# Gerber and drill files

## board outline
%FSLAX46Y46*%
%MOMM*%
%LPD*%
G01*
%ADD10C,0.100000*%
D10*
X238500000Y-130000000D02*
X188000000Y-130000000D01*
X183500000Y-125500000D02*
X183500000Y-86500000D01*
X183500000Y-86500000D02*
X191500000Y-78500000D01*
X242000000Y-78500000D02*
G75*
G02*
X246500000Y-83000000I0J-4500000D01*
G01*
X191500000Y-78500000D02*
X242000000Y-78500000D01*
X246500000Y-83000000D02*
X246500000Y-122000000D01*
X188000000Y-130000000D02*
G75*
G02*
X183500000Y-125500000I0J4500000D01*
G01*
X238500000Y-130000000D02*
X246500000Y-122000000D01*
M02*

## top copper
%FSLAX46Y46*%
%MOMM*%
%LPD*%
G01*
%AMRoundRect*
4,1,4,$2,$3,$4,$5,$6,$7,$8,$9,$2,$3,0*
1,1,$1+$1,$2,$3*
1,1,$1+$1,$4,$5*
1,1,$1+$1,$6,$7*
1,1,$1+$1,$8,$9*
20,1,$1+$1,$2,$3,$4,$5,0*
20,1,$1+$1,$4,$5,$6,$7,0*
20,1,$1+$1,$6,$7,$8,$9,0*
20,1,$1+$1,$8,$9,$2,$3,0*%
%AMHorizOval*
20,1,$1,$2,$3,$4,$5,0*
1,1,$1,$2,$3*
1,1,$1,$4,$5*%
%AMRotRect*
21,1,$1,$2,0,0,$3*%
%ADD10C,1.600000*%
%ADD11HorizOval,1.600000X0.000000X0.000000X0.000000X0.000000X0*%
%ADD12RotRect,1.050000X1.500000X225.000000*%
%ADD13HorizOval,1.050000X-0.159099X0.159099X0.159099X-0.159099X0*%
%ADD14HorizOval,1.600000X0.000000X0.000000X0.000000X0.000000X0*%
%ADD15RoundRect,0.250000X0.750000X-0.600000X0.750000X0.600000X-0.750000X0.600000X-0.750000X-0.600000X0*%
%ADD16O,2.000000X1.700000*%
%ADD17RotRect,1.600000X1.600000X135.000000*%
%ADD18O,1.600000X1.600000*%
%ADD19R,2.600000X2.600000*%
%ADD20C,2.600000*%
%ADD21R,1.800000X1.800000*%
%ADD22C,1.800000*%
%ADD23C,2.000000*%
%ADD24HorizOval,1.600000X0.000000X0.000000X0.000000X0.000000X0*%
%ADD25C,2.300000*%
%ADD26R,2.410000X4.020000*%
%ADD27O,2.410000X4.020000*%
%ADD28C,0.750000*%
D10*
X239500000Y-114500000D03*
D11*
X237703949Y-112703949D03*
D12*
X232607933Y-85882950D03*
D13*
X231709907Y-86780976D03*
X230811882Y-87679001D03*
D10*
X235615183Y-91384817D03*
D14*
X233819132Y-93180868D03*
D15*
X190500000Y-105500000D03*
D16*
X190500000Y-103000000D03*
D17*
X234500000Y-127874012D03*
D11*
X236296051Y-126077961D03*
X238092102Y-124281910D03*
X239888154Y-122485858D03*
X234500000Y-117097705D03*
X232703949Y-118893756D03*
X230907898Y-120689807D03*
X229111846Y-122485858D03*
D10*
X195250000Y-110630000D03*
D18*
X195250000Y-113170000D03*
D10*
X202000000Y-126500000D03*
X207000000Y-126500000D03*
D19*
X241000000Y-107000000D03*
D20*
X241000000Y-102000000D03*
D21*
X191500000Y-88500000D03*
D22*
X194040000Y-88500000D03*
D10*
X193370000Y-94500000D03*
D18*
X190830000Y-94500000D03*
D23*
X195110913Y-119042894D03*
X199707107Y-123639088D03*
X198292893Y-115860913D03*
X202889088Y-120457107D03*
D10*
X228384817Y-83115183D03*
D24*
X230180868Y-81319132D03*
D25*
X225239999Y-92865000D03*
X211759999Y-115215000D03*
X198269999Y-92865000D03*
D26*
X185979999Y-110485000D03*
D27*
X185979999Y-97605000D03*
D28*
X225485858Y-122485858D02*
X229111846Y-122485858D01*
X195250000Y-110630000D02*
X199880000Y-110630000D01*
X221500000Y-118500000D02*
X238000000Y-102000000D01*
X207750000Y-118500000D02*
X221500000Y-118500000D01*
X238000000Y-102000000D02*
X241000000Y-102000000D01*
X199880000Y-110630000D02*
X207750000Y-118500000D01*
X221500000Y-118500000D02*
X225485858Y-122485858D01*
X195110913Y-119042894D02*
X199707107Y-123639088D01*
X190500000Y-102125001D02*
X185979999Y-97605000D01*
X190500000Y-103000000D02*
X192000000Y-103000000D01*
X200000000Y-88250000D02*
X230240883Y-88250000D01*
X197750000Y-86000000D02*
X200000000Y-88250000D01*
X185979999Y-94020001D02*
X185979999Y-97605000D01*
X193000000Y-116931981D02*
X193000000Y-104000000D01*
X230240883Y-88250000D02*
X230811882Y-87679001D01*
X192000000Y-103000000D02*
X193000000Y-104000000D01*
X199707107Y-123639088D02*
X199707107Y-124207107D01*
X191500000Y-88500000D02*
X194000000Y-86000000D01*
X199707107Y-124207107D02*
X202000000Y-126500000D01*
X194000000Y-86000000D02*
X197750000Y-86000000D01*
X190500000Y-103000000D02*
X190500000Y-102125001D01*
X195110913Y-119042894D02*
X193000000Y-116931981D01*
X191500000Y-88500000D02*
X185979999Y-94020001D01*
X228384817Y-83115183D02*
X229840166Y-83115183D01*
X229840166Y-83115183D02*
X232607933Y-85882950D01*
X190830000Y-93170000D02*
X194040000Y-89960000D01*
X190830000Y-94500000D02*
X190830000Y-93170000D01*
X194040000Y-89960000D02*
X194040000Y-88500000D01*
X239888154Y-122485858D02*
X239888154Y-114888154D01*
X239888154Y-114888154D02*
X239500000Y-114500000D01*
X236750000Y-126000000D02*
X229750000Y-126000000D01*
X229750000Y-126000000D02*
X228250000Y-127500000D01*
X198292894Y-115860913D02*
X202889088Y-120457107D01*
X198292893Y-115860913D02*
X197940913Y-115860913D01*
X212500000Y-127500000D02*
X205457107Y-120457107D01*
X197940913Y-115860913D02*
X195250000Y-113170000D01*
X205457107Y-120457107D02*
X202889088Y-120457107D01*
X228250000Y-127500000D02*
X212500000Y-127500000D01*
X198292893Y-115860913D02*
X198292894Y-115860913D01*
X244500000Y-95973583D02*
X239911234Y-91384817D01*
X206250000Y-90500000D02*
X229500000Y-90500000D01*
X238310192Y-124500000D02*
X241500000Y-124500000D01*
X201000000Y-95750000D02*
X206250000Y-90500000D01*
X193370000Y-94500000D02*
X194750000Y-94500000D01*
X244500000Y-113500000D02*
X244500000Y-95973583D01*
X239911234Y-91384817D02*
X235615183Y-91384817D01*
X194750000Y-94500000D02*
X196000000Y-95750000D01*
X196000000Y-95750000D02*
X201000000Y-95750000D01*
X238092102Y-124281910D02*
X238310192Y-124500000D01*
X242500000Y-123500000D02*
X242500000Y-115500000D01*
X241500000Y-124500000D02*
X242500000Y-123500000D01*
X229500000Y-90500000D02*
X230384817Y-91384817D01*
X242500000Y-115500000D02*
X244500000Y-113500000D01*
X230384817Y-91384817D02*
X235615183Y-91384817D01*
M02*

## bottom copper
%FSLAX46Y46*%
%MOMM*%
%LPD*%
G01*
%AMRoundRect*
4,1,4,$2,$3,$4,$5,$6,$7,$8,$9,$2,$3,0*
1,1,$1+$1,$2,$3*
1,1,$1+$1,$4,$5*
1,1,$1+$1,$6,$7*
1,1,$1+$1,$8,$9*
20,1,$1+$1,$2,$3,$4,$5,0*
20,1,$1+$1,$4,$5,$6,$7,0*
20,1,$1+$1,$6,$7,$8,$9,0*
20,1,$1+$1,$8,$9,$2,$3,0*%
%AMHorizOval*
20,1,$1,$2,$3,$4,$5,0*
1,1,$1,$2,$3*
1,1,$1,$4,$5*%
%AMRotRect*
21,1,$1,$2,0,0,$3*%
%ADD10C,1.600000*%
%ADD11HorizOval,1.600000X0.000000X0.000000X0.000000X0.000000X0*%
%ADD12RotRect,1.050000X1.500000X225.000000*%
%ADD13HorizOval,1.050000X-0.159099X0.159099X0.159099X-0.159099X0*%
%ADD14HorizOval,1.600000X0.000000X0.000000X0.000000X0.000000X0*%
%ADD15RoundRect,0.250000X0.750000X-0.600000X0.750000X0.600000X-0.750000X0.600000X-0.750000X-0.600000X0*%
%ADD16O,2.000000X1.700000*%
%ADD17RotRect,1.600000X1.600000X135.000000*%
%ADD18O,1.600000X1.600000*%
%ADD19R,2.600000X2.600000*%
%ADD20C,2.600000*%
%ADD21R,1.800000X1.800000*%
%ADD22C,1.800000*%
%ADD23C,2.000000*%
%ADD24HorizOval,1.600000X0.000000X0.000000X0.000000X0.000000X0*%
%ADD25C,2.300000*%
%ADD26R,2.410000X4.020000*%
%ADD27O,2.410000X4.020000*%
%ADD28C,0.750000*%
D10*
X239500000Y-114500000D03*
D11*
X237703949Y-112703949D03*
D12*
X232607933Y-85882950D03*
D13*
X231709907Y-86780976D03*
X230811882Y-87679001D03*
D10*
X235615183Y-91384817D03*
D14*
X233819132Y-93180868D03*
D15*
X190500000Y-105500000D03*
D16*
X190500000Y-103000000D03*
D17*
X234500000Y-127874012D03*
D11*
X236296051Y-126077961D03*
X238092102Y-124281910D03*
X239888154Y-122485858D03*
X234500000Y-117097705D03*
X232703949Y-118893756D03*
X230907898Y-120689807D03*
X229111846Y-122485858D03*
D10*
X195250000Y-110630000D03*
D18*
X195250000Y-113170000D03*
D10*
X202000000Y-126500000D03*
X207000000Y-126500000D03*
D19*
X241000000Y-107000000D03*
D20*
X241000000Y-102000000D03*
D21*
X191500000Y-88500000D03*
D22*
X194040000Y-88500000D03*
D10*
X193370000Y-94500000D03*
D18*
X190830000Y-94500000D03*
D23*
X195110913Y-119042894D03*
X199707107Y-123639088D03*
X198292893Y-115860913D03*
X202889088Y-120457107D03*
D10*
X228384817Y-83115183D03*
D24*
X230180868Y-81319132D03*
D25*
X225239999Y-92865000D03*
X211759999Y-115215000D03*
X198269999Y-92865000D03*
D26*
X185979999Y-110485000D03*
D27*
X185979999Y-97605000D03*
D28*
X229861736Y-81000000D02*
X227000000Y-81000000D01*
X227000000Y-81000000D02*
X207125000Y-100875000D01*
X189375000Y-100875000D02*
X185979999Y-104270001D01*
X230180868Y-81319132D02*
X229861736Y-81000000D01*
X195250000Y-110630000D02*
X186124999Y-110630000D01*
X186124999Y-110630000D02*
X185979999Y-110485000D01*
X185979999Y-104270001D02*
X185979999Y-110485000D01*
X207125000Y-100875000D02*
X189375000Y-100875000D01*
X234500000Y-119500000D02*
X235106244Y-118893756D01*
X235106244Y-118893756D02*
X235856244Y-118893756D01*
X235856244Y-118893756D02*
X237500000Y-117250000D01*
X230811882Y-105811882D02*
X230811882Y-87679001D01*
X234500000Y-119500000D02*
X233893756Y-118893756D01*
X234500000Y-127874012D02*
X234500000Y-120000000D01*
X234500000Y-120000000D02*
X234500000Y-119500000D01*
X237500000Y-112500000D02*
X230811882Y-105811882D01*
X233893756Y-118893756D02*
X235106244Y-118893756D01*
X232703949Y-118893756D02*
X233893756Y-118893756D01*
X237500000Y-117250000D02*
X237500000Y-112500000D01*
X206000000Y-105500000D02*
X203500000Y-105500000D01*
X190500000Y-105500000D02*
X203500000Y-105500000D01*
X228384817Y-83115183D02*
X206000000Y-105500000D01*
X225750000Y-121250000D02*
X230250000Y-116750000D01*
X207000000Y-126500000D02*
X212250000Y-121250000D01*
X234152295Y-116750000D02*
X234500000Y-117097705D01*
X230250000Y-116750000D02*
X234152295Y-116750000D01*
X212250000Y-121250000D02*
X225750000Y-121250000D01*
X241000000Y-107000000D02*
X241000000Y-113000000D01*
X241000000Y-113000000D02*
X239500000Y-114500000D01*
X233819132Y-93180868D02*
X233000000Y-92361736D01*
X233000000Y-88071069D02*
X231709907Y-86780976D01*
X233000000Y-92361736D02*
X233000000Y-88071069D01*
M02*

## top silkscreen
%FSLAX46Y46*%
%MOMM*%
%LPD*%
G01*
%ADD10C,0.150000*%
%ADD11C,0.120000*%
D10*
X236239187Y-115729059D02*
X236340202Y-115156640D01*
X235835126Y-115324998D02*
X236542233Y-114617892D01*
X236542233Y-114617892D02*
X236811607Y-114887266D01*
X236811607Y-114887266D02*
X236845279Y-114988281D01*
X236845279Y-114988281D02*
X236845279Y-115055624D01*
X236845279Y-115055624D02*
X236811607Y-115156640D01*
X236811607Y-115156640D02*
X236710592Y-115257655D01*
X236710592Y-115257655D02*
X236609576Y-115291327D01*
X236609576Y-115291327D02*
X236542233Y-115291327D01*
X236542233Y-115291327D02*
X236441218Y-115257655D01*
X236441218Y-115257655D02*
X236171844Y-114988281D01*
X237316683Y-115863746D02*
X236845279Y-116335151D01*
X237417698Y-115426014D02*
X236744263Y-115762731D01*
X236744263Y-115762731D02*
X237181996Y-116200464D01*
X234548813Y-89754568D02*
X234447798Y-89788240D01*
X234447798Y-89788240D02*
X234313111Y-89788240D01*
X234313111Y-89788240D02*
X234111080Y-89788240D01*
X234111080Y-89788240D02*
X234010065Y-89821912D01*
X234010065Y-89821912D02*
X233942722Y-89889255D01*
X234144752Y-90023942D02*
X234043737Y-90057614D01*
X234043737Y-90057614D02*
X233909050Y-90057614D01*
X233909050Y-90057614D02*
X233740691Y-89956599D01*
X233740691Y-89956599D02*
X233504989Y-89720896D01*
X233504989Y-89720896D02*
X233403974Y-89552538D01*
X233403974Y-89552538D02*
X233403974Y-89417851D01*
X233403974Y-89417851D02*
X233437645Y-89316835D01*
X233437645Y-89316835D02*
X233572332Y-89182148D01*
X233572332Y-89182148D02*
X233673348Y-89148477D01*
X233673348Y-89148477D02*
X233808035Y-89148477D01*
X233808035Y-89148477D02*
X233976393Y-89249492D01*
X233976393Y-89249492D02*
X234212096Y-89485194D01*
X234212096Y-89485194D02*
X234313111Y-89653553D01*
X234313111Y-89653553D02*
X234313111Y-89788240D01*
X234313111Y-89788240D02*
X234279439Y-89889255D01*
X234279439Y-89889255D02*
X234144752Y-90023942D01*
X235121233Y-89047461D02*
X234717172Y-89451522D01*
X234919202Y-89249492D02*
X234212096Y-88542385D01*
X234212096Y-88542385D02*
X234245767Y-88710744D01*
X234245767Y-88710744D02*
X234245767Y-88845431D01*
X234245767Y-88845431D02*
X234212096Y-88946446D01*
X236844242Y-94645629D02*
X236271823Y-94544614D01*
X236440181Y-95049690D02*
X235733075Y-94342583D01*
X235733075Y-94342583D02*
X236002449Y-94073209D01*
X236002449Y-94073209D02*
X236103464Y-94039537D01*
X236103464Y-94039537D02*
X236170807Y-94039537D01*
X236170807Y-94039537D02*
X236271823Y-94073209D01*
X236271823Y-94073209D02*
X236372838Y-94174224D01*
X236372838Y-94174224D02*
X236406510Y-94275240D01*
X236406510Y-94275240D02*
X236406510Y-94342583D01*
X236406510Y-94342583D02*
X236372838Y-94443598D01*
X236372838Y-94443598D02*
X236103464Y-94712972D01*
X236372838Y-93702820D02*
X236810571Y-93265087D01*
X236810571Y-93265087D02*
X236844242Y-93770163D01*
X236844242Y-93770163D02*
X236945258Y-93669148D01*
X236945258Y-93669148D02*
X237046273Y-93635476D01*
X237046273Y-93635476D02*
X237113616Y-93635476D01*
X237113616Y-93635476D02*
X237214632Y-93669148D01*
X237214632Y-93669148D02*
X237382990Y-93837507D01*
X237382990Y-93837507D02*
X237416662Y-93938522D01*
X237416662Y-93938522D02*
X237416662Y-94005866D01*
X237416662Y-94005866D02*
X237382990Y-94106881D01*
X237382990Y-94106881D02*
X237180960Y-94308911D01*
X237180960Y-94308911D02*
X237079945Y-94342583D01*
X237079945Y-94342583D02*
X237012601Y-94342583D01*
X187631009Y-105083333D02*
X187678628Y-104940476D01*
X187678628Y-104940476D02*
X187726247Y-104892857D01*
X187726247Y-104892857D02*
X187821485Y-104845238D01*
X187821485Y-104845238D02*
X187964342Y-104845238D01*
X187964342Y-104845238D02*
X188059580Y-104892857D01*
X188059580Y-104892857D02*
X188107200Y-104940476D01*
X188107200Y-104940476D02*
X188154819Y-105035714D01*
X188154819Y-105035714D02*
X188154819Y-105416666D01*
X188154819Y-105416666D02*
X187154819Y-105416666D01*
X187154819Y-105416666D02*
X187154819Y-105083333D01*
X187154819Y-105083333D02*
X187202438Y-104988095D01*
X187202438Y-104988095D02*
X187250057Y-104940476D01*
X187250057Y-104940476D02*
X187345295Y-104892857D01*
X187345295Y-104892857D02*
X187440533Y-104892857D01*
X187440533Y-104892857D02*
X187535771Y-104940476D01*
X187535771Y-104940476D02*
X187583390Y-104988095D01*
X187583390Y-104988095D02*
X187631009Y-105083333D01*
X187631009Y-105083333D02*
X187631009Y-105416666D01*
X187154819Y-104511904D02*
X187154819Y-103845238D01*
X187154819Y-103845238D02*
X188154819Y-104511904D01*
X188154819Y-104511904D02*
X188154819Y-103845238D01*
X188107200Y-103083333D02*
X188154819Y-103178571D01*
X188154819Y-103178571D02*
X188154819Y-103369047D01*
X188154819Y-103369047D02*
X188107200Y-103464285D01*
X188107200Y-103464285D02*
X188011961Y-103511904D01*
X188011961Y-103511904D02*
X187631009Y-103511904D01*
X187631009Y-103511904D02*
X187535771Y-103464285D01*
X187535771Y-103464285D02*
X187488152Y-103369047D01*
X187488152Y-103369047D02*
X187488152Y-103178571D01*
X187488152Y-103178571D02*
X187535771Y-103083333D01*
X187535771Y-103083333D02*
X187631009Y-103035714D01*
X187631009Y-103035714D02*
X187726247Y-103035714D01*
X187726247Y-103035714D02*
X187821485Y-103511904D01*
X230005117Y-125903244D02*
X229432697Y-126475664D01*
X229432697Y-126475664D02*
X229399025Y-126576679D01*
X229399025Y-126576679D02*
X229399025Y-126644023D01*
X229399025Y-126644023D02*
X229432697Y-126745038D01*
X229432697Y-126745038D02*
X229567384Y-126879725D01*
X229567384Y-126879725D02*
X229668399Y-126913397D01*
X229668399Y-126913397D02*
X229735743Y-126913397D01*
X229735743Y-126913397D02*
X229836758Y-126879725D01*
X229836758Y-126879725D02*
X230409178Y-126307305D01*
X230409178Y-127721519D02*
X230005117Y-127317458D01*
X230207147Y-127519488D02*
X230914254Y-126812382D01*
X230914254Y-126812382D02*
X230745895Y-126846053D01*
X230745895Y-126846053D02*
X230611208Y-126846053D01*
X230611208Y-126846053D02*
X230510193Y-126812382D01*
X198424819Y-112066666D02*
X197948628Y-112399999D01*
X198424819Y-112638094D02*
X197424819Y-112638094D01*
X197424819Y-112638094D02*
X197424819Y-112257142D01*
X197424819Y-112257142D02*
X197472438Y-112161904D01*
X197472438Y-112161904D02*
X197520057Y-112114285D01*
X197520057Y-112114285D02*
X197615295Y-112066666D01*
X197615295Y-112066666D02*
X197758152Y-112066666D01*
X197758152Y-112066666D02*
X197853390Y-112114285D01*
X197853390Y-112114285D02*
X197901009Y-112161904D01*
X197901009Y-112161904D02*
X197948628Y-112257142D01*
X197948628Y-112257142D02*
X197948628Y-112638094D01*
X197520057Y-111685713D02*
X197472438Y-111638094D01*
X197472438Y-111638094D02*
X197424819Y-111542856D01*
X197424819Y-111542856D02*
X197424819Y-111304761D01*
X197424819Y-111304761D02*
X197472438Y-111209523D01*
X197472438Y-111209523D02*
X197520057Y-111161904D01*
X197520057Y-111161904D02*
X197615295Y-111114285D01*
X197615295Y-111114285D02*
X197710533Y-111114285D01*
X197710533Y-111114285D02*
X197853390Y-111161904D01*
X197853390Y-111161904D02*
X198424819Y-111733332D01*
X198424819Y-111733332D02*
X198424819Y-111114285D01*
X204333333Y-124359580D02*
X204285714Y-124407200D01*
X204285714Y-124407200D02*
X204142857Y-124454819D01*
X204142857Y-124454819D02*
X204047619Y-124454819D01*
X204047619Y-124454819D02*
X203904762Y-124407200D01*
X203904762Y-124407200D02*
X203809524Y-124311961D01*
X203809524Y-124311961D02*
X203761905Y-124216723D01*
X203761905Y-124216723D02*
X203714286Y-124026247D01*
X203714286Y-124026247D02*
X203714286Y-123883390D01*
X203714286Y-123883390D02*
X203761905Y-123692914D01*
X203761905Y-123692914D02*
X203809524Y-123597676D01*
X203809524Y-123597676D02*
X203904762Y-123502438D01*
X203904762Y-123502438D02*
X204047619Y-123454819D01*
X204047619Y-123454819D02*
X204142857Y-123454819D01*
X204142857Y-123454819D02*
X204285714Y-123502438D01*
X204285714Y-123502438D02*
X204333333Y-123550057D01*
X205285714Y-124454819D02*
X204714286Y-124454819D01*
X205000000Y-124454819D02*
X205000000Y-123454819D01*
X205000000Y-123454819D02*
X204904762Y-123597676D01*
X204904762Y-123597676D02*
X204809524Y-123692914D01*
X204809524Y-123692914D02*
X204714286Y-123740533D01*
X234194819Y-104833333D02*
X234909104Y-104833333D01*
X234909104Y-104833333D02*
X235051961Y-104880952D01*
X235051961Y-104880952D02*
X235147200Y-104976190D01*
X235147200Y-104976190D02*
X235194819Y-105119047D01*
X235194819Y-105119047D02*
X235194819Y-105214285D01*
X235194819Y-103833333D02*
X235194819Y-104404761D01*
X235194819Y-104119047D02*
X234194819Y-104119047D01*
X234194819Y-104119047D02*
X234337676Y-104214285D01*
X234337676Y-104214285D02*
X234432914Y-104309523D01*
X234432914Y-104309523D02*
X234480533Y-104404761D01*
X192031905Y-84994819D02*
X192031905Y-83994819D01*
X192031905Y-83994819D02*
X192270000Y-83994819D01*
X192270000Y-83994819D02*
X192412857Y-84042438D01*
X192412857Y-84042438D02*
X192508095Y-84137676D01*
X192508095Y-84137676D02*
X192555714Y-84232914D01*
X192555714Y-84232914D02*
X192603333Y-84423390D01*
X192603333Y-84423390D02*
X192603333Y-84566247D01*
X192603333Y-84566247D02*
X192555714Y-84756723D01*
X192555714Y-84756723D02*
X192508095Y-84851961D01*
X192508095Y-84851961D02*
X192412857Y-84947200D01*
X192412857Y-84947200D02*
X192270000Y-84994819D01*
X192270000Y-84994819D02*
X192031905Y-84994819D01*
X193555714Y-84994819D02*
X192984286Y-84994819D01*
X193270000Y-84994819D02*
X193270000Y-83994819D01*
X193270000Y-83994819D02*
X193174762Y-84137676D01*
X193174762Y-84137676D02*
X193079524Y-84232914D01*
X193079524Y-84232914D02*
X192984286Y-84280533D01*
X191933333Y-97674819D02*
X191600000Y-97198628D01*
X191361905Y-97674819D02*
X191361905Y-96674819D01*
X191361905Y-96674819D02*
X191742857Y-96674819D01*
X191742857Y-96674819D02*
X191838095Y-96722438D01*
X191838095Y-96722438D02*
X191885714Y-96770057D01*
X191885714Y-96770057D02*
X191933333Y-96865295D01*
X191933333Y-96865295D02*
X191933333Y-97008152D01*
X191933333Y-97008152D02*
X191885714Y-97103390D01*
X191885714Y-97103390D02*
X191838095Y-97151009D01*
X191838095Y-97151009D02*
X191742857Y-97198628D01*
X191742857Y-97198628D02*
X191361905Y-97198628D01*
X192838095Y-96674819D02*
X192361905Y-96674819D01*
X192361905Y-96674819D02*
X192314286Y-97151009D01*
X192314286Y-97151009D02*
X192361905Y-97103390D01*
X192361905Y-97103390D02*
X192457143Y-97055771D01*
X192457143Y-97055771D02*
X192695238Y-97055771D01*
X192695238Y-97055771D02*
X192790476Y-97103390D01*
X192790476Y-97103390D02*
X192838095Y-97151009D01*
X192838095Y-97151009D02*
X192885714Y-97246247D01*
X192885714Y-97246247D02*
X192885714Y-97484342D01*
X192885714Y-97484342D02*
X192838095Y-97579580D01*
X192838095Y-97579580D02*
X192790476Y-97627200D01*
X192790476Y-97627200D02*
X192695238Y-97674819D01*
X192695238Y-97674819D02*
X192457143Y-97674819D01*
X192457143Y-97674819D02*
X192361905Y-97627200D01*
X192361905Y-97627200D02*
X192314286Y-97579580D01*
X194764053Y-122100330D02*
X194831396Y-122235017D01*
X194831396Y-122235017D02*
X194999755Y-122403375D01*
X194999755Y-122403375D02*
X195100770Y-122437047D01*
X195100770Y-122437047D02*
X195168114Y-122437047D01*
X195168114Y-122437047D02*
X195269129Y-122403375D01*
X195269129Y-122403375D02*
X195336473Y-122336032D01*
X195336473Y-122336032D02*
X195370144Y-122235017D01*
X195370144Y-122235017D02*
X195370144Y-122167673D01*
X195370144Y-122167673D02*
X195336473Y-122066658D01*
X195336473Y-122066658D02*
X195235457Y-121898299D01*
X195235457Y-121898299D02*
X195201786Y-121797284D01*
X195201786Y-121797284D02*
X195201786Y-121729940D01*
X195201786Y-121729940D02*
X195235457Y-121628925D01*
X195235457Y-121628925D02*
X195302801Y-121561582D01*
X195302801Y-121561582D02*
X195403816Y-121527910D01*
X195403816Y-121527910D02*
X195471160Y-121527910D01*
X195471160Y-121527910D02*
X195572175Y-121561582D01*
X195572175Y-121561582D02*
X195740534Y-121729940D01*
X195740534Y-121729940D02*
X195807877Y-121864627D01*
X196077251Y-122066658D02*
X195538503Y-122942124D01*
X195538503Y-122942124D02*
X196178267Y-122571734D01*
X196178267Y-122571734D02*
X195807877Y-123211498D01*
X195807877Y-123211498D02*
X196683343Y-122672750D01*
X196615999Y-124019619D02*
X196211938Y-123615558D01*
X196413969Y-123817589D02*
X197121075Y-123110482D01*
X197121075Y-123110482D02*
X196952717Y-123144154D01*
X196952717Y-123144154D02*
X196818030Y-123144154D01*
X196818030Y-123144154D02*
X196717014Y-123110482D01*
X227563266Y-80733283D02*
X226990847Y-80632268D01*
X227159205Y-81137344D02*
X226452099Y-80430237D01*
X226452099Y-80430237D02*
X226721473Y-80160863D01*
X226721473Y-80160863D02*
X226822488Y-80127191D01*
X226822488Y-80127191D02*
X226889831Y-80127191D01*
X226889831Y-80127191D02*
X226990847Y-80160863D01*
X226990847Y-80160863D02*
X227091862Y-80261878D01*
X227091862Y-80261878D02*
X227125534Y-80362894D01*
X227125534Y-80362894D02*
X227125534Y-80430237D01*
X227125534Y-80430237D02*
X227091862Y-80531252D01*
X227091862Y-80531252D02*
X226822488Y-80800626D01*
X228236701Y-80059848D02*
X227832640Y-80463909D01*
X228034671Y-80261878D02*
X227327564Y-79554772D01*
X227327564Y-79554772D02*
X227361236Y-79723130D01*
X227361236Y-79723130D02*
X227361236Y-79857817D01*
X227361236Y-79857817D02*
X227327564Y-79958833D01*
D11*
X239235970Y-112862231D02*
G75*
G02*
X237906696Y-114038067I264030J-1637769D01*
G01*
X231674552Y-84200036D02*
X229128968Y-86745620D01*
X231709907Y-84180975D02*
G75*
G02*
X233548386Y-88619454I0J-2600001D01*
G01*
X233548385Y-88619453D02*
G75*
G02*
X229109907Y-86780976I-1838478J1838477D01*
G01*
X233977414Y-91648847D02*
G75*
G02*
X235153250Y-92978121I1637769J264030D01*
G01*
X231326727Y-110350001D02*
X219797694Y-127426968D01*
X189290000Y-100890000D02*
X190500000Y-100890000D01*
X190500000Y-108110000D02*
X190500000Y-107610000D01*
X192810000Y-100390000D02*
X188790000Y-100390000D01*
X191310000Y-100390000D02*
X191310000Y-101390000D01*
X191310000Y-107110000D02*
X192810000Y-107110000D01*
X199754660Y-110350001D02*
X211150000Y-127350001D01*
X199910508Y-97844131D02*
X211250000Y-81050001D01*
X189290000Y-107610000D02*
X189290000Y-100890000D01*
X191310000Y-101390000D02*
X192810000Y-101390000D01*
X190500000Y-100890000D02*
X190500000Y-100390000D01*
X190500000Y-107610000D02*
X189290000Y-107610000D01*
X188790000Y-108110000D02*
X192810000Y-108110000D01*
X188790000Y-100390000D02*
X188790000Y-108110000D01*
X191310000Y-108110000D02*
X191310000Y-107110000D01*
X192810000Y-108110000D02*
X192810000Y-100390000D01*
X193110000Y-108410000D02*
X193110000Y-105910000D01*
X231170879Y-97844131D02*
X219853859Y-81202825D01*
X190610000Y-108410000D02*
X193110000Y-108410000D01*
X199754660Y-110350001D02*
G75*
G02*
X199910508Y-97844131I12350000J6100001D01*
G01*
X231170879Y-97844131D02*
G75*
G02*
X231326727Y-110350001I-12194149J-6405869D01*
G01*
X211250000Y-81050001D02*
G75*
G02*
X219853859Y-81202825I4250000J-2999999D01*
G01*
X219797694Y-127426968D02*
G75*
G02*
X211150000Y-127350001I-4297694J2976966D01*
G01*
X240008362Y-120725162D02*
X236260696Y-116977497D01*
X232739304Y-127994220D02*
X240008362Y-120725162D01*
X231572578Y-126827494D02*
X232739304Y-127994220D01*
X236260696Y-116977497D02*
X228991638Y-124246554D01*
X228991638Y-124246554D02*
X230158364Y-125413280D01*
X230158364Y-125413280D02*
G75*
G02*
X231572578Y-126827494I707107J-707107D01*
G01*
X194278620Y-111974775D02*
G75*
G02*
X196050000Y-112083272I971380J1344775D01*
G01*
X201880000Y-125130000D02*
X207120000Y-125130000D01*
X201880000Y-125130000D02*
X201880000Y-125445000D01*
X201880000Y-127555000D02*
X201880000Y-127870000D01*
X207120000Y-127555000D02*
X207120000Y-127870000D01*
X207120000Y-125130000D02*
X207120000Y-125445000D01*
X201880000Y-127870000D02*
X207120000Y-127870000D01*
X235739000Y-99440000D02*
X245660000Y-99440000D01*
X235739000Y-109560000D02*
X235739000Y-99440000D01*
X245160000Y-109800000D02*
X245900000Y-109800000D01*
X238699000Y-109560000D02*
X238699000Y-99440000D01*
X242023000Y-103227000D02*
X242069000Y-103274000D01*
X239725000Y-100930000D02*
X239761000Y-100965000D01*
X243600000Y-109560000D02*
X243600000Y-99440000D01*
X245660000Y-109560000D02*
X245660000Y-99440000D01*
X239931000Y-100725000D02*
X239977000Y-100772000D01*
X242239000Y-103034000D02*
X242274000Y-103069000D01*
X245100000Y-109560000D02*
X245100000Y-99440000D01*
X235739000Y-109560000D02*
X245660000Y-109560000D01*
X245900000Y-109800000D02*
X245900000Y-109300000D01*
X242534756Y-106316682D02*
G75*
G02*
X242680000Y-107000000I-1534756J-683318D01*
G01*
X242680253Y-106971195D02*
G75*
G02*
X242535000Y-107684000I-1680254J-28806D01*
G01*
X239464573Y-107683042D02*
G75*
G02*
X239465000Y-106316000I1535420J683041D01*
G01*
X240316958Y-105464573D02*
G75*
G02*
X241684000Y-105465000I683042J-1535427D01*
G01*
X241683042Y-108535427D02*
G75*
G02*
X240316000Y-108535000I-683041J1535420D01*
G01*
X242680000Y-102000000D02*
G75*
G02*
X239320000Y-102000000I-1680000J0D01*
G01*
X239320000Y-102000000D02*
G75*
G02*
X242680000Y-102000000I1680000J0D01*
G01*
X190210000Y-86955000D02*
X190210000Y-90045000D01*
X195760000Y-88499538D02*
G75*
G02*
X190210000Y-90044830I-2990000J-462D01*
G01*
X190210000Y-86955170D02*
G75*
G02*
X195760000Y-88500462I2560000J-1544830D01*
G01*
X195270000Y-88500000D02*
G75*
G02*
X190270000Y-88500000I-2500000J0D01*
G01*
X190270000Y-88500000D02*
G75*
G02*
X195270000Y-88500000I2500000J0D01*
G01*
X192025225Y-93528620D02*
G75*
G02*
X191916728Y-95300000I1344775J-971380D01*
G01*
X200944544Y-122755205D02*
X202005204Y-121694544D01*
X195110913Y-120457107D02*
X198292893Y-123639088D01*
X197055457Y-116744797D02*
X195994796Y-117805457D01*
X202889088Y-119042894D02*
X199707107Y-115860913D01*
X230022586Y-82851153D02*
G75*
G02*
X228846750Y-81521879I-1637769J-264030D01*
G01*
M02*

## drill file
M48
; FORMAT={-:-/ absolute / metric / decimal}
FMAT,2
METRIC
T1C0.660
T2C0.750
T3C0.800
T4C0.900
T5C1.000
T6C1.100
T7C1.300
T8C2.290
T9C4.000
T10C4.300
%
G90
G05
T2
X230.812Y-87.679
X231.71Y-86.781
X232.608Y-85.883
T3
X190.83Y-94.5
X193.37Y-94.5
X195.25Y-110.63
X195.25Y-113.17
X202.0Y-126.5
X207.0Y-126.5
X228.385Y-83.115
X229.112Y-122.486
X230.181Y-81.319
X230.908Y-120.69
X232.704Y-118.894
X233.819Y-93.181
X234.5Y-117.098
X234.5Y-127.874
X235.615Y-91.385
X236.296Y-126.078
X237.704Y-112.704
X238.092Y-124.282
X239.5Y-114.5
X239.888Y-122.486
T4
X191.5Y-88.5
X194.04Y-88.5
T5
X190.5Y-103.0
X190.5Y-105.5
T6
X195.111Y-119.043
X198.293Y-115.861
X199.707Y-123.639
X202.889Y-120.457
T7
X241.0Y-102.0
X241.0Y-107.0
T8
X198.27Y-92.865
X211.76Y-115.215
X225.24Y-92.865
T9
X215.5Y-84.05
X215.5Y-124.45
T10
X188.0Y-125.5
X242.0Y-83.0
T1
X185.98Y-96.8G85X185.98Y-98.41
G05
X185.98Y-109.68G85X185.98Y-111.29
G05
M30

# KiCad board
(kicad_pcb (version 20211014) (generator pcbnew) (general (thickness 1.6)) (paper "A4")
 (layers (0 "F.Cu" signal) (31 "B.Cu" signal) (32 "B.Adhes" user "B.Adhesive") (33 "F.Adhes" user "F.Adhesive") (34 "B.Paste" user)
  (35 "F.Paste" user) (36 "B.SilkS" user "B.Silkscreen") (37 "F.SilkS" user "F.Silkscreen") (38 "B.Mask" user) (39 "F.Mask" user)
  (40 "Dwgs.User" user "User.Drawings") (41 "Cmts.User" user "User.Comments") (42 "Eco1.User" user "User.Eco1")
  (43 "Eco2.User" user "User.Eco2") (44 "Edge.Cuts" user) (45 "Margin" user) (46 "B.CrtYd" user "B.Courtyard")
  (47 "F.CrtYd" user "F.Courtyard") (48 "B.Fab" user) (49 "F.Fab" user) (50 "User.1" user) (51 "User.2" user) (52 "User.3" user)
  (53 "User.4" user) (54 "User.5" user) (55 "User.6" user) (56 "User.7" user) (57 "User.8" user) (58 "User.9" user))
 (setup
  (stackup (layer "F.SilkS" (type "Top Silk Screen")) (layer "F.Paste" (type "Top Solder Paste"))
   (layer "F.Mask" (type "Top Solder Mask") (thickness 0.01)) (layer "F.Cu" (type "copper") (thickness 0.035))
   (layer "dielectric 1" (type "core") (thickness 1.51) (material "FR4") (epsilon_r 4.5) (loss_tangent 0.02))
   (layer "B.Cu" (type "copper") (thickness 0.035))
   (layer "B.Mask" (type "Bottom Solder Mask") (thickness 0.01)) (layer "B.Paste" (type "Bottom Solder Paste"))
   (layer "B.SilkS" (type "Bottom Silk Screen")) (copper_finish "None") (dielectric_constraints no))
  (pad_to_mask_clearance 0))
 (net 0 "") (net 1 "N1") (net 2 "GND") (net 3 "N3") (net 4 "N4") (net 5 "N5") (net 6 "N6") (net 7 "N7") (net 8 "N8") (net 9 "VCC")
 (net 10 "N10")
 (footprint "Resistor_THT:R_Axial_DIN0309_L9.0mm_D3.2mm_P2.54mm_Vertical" (layer "F.Cu") (at 239.5 114.5 135)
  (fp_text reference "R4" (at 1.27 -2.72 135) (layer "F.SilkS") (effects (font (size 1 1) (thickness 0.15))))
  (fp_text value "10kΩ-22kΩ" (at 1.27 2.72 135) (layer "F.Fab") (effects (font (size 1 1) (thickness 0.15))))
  (fp_arc (start 1.344775 0.97138) (mid -1.655812 -0.101418) (end 1.453272 -0.8) (layer "F.SilkS") (width 0.12))
  (pad "1" thru_hole circle (at 0 0 135) (size 1.6 1.6) (drill 0.8) (layers *.Cu *.Mask) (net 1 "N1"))
  (pad "2" thru_hole oval (at 2.54 0 135) (size 1.6 1.6) (drill 0.8) (layers *.Cu *.Mask) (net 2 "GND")))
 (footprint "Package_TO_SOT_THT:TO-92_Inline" (layer "F.Cu") (at 232.607933 85.88295 -135)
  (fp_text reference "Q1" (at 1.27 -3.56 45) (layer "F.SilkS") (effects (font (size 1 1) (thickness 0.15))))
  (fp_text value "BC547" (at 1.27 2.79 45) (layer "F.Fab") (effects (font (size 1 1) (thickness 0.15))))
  (fp_line (start -0.53 1.85) (end 3.07 1.85) (layer "F.SilkS") (width 0.12))
  (fp_arc (start -0.568478 1.838478) (mid -1.132087 -0.994977) (end 1.27 -2.6) (layer "F.SilkS") (width 0.12))
  (fp_arc (start 1.27 -2.6) (mid 3.672087 -0.994977) (end 3.108478 1.838478) (layer "F.SilkS") (width 0.12))
  (pad "1" thru_hole rect (at 0 0 225) (size 1.05 1.5) (drill 0.75) (layers *.Cu *.Mask) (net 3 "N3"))
  (pad "2" thru_hole oval (at 1.27 0 225) (size 1.05 1.5) (drill 0.75) (layers *.Cu *.Mask) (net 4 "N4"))
  (pad "3" thru_hole oval (at 2.54 0 225) (size 1.05 1.5) (drill 0.75) (layers *.Cu *.Mask) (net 2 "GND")))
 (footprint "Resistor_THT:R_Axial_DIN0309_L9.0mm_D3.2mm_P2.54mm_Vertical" (layer "F.Cu") (at 235.615183 91.384817 -135)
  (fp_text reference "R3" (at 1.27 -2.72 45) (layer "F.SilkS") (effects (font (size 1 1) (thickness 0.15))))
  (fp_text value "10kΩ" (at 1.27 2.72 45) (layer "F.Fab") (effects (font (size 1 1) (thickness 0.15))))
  (fp_arc (start 1.344775 0.97138) (mid -1.655812 -0.101418) (end 1.453272 -0.8) (layer "F.SilkS") (width 0.12))
  (pad "1" thru_hole circle (at 0 0 225) (size 1.6 1.6) (drill 0.8) (layers *.Cu *.Mask) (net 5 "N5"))
  (pad "2" thru_hole oval (at 2.54 0 225) (size 1.6 1.6) (drill 0.8) (layers *.Cu *.Mask) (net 4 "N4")))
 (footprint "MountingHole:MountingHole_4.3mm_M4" (layer "F.Cu") (at 242 83)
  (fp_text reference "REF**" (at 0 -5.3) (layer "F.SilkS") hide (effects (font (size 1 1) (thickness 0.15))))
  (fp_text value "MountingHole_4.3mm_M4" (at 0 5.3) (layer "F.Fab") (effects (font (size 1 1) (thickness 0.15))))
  (pad "" np_thru_hole circle (at 0 0) (size 4.3 4.3) (drill 4.3) (layers *.Cu *.Mask)))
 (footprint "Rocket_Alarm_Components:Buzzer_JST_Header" (layer "F.Cu") (at 190.5 105.5 90)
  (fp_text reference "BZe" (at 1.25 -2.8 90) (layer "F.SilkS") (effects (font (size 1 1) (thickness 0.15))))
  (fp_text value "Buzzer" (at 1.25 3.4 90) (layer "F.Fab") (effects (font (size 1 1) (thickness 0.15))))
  (fp_line (start -4.850001 40.826727) (end -21.926968 29.297694) (layer "F.SilkS") (width 0.12))
  (fp_line (start 4.61 -1.21) (end 4.61 0) (layer "F.SilkS") (width 0.12))
  (fp_line (start -2.61 0) (end -2.11 0) (layer "F.SilkS") (width 0.12))
  (fp_line (start 5.11 2.31) (end 5.11 -1.71) (layer "F.SilkS") (width 0.12))
  (fp_line (start 5.11 0.81) (end 4.11 0.81) (layer "F.SilkS") (width 0.12))
  (fp_line (start -1.61 0.81) (end -1.61 2.31) (layer "F.SilkS") (width 0.12))
  (fp_line (start -4.850001 9.25466) (end -21.850001 20.65) (layer "F.SilkS") (width 0.12))
  (fp_line (start 7.655869 9.410508) (end 24.449999 20.75) (layer "F.SilkS") (width 0.12))
  (fp_line (start -2.11 -1.21) (end 4.61 -1.21) (layer "F.SilkS") (width 0.12))
  (fp_line (start 4.11 0.81) (end 4.11 2.31) (layer "F.SilkS") (width 0.12))
  (fp_line (start 4.61 0) (end 5.11 0) (layer "F.SilkS") (width 0.12))
  (fp_line (start -2.11 0) (end -2.11 -1.21) (layer "F.SilkS") (width 0.12))
  (fp_line (start -2.61 -1.71) (end -2.61 2.31) (layer "F.SilkS") (width 0.12))
  (fp_line (start 5.11 -1.71) (end -2.61 -1.71) (layer "F.SilkS") (width 0.12))
  (fp_line (start -2.61 0.81) (end -1.61 0.81) (layer "F.SilkS") (width 0.12))
  (fp_line (start -2.61 2.31) (end 5.11 2.31) (layer "F.SilkS") (width 0.12))
  (fp_line (start -2.91 2.61) (end -0.41 2.61) (layer "F.SilkS") (width 0.12))
  (fp_line (start 7.655869 40.670879) (end 24.297175 29.353859) (layer "F.SilkS") (width 0.12))
  (fp_line (start -2.91 0.11) (end -2.91 2.61) (layer "F.SilkS") (width 0.12))
  (fp_arc (start -4.850001 9.25466) (mid 1.421642 7.831387) (end 7.655869 9.410508) (layer "F.SilkS") (width 0.12))
  (fp_arc (start 7.655869 40.670879) (mid 1.421642 42.25) (end -4.850001 40.826727) (layer "F.SilkS") (width 0.12))
  (fp_arc (start 24.449999 20.75) (mid 26.651342 25.092388) (end 24.297175 29.353859) (layer "F.SilkS") (width 0.12))
  (fp_arc (start -21.926968 29.297694) (mid -24.177844 24.953471) (end -21.850001 20.65) (layer "F.SilkS") (width 0.12))
  (pad "" np_thru_hole circle (at 21.449999 25 90) (size 4 4) (drill 4) (layers F&B.Cu *.Mask))
  (pad "" np_thru_hole circle (at -18.950001 25 90) (size 4 4) (drill 4) (layers F&B.Cu *.Mask))
  (pad "1" thru_hole roundrect (at 0 0 90) (size 1.7 2) (drill 1) (layers *.Cu *.Mask) (roundrect_rratio 0.147059) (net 3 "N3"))
  (pad "2" thru_hole oval (at 2.5 0 90) (size 1.7 2) (drill 1) (layers *.Cu *.Mask) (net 2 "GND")))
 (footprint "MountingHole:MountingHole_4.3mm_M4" (layer "F.Cu") (at 188 125.5)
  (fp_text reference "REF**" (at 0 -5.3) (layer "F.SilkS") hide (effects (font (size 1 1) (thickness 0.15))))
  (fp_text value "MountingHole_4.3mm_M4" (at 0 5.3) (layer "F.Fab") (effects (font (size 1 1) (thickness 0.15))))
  (pad "" np_thru_hole circle (at 0 0) (size 4.3 4.3) (drill 4.3) (layers *.Cu *.Mask)))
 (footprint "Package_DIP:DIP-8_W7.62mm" (layer "F.Cu") (at 234.5 127.874012 135)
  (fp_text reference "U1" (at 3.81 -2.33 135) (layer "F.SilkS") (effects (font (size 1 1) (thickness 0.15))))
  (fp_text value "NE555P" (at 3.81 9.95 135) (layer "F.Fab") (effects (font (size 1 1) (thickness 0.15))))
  (fp_line (start 1.16 8.95) (end 6.46 8.95) (layer "F.SilkS") (width 0.12))
  (fp_line (start 1.16 -1.33) (end 1.16 8.95) (layer "F.SilkS") (width 0.12))
  (fp_line (start 2.81 -1.33) (end 1.16 -1.33) (layer "F.SilkS") (width 0.12))
  (fp_line (start 6.46 8.95) (end 6.46 -1.33) (layer "F.SilkS") (width 0.12))
  (fp_line (start 6.46 -1.33) (end 4.81 -1.33) (layer "F.SilkS") (width 0.12))
  (fp_arc (start 4.81 -1.33) (mid 3.81 -0.33) (end 2.81 -1.33) (layer "F.SilkS") (width 0.12))
  (pad "1" thru_hole rect (at 0 0 135) (size 1.6 1.6) (drill 0.8) (layers *.Cu *.Mask) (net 2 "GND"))
  (pad "2" thru_hole oval (at 0 2.54 135) (size 1.6 1.6) (drill 0.8) (layers *.Cu *.Mask) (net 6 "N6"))
  (pad "3" thru_hole oval (at 0 5.08 135) (size 1.6 1.6) (drill 0.8) (layers *.Cu *.Mask) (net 5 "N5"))
  (pad "4" thru_hole oval (at 0 7.62 135) (size 1.6 1.6) (drill 0.8) (layers *.Cu *.Mask) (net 1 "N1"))
  (pad "5" thru_hole oval (at 7.62 7.62 135) (size 1.6 1.6) (drill 0.8) (layers *.Cu *.Mask) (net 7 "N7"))
  (pad "6" thru_hole oval (at 7.62 5.08 135) (size 1.6 1.6) (drill 0.8) (layers *.Cu *.Mask) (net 2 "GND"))
  (pad "7" thru_hole oval (at 7.62 2.54 135) (size 1.6 1.6) (drill 0.8) (layers *.Cu *.Mask) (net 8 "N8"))
  (pad "8" thru_hole oval (at 7.62 0 135) (size 1.6 1.6) (drill 0.8) (layers *.Cu *.Mask) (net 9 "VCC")))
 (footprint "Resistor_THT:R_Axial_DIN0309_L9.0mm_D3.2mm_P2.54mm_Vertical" (layer "F.Cu") (at 195.25 110.63 -90)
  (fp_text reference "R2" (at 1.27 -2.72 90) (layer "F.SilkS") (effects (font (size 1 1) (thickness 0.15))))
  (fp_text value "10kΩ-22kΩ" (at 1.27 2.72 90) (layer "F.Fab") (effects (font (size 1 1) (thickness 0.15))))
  (fp_arc (start 1.344775 0.97138) (mid -1.655812 -0.101418) (end 1.453272 -0.8) (layer "F.SilkS") (width 0.12))
  (pad "1" thru_hole circle (at 0 0 270) (size 1.6 1.6) (drill 0.8) (layers *.Cu *.Mask) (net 9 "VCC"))
  (pad "2" thru_hole oval (at 2.54 0 270) (size 1.6 1.6) (drill 0.8) (layers *.Cu *.Mask) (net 6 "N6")))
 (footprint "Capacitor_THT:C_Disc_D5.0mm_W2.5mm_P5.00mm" (layer "F.Cu") (at 202 126.5)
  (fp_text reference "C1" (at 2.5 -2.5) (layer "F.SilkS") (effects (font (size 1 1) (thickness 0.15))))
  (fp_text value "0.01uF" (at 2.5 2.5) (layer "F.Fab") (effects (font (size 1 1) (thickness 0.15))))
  (fp_line (start -0.12 -1.37) (end 5.12 -1.37) (layer "F.SilkS") (width 0.12))
  (fp_line (start -0.12 -1.37) (end -0.12 -1.055) (layer "F.SilkS") (width 0.12))
  (fp_line (start -0.12 1.055) (end -0.12 1.37) (layer "F.SilkS") (width 0.12))
  (fp_line (start 5.12 1.055) (end 5.12 1.37) (layer "F.SilkS") (width 0.12))
  (fp_line (start 5.12 -1.37) (end 5.12 -1.055) (layer "F.SilkS") (width 0.12))
  (fp_line (start -0.12 1.37) (end 5.12 1.37) (layer "F.SilkS") (width 0.12))
  (pad "1" thru_hole circle (at 0 0) (size 1.6 1.6) (drill 0.8) (layers *.Cu *.Mask) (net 2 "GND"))
  (pad "2" thru_hole circle (at 5 0) (size 1.6 1.6) (drill 0.8) (layers *.Cu *.Mask) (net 7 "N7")))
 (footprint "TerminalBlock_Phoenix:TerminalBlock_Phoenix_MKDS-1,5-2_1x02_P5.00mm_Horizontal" (layer "F.Cu") (at 241 107 90)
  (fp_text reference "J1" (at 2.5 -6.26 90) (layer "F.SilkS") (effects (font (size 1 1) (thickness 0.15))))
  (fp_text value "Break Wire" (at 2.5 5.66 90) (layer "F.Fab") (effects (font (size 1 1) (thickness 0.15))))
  (fp_line (start 7.56 -5.261) (end 7.56 4.66) (layer "F.SilkS") (width 0.12))
  (fp_line (start -2.56 -5.261) (end 7.56 -5.261) (layer "F.SilkS") (width 0.12))
  (fp_line (start -2.8 4.16) (end -2.8 4.9) (layer "F.SilkS") (width 0.12))
  (fp_line (start -2.56 -2.301) (end 7.56 -2.301) (layer "F.SilkS") (width 0.12))
  (fp_line (start 3.773 1.023) (end 3.726 1.069) (layer "F.SilkS") (width 0.12))
  (fp_line (start 6.07 -1.275) (end 6.035 -1.239) (layer "F.SilkS") (width 0.12))
  (fp_line (start -2.56 2.6) (end 7.56 2.6) (layer "F.SilkS") (width 0.12))
  (fp_line (start -2.56 4.66) (end 7.56 4.66) (layer "F.SilkS") (width 0.12))
  (fp_line (start 6.275 -1.069) (end 6.228 -1.023) (layer "F.SilkS") (width 0.12))
  (fp_line (start 3.966 1.239) (end 3.931 1.274) (layer "F.SilkS") (width 0.12))
  (fp_line (start -2.56 4.1) (end 7.56 4.1) (layer "F.SilkS") (width 0.12))
  (fp_line (start -2.56 -5.261) (end -2.56 4.66) (layer "F.SilkS") (width 0.12))
  (fp_line (start -2.8 4.9) (end -2.3 4.9) (layer "F.SilkS") (width 0.12))
  (fp_arc (start 0.683318 1.534756) (mid 0.349292 1.643288) (end 0 1.68) (layer "F.SilkS") (width 0.12))
  (fp_arc (start 0.028805 1.680253) (mid -0.335551 1.646659) (end -0.684 1.535) (layer "F.SilkS") (width 0.12))
  (fp_arc (start -0.683042 -1.535427) (mid 0.000524 -1.680501) (end 0.684 -1.535) (layer "F.SilkS") (width 0.12))
  (fp_arc (start 1.535427 -0.683042) (mid 1.680501 0.000524) (end 1.535 0.684) (layer "F.SilkS") (width 0.12))
  (fp_arc (start -1.535427 0.683042) (mid -1.680501 -0.000524) (end -1.535 -0.684) (layer "F.SilkS") (width 0.12))
  (fp_circle (center 5 0) (end 6.68 0) (layer "F.SilkS") (width 0.12) (fill none))
  (pad "1" thru_hole rect (at 0 0 90) (size 2.6 2.6) (drill 1.3) (layers *.Cu *.Mask) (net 1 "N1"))
  (pad "2" thru_hole circle (at 5 0 90) (size 2.6 2.6) (drill 1.3) (layers *.Cu *.Mask) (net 9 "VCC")))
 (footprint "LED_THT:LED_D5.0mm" (layer "F.Cu") (at 191.5 88.5)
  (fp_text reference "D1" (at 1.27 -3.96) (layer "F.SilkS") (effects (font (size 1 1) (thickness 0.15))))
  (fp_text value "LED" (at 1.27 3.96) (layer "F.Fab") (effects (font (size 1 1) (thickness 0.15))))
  (fp_line (start -1.29 -1.545) (end -1.29 1.545) (layer "F.SilkS") (width 0.12))
  (fp_arc (start 4.26 -0.000462) (mid 2.072002 2.880433) (end -1.29 1.54483) (layer "F.SilkS") (width 0.12))
  (fp_arc (start -1.29 -1.54483) (mid 2.072002 -2.880433) (end 4.26 0.000462) (layer "F.SilkS") (width 0.12))
  (fp_circle (center 1.27 0) (end 3.77 0) (layer "F.SilkS") (width 0.12) (fill none))
  (pad "1" thru_hole rect (at 0 0) (size 1.8 1.8) (drill 0.9) (layers *.Cu *.Mask) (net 2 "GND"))
  (pad "2" thru_hole circle (at 2.54 0) (size 1.8 1.8) (drill 0.9) (layers *.Cu *.Mask) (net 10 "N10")))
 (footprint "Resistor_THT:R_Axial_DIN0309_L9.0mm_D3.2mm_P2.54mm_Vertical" (layer "F.Cu") (at 193.37 94.5 180)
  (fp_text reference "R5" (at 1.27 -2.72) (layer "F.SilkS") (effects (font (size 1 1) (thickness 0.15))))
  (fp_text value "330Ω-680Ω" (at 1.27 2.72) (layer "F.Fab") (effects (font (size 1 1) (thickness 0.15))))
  (fp_arc (start 1.344775 0.97138) (mid -1.655812 -0.101418) (end 1.453272 -0.8) (layer "F.SilkS") (width 0.12))
  (pad "1" thru_hole circle (at 0 0 180) (size 1.6 1.6) (drill 0.8) (layers *.Cu *.Mask) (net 5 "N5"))
  (pad "2" thru_hole oval (at 2.54 0 180) (size 1.6 1.6) (drill 0.8) (layers *.Cu *.Mask) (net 10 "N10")))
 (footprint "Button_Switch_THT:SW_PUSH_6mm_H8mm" (layer "F.Cu") (at 199.707107 123.639088 135)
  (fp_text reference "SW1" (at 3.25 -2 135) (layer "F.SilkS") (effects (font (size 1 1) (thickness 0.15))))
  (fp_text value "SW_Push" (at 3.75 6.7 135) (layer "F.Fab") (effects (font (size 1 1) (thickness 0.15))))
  (fp_line (start -0.25 1.5) (end -0.25 3) (layer "F.SilkS") (width 0.12))
  (fp_line (start 5.5 -1) (end 1 -1) (layer "F.SilkS") (width 0.12))
  (fp_line (start 6.75 3) (end 6.75 1.5) (layer "F.SilkS") (width 0.12))
  (fp_line (start 1 5.5) (end 5.5 5.5) (layer "F.SilkS") (width 0.12))
  (pad "1" thru_hole circle (at 6.5 0 225) (size 2 2) (drill 1.1) (layers *.Cu *.Mask) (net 2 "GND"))
  (pad "1" thru_hole circle (at 0 0 225) (size 2 2) (drill 1.1) (layers *.Cu *.Mask) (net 2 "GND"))
  (pad "2" thru_hole circle (at 6.5 4.5 225) (size 2 2) (drill 1.1) (layers *.Cu *.Mask) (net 6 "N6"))
  (pad "2" thru_hole circle (at 0 4.5 225) (size 2 2) (drill 1.1) (layers *.Cu *.Mask) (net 6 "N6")))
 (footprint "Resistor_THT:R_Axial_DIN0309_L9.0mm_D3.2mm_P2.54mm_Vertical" (layer "F.Cu") (at 228.384817 83.115183 45)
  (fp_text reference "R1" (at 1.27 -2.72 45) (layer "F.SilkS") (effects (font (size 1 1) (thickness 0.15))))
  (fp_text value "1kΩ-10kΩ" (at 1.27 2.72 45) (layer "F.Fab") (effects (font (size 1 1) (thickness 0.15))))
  (fp_arc (start 1.344775 0.97138) (mid -1.655812 -0.101418) (end 1.453272 -0.8) (layer "F.SilkS") (width 0.12))
  (pad "1" thru_hole circle (at 0 0 45) (size 1.6 1.6) (drill 0.8) (layers *.Cu *.Mask) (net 3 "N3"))
  (pad "2" thru_hole oval (at 2.54 0 45) (size 1.6 1.6) (drill 0.8) (layers *.Cu *.Mask) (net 9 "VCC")))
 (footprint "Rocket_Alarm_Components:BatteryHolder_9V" (layer "B.Cu") (at 185.979999 110.485)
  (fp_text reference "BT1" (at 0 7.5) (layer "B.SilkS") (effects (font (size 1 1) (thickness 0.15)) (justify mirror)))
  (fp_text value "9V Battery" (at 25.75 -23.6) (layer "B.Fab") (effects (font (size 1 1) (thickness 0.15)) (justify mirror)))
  (pad "" np_thru_hole circle (at 39.26 -17.62) (size 2.3 2.3) (drill 2.29) (layers *.Cu *.Mask))
  (pad "" np_thru_hole circle (at 25.78 4.73) (size 2.3 2.3) (drill 2.29) (layers *.Cu *.Mask))
  (pad "" np_thru_hole circle (at 12.29 -17.62) (size 2.3 2.3) (drill 2.29) (layers *.Cu *.Mask))
  (pad "1" thru_hole rect (at 0 0) (size 2.41 4.02) (drill oval 0.66 2.27) (layers *.Cu *.Mask) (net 9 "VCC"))
  (pad "2" thru_hole oval (at 0 -12.88) (size 2.41 4.02) (drill oval 0.66 2.27) (layers *.Cu *.Mask) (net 2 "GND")))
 (gr_line (start 238.5 130) (end 188 130) (layer "Edge.Cuts") (width 0.1))
 (gr_line (start 183.5 125.5) (end 183.5 86.5) (layer "Edge.Cuts") (width 0.1))
 (gr_line (start 183.5 86.5) (end 191.5 78.5) (layer "Edge.Cuts") (width 0.1))
 (gr_arc (start 242 78.5) (mid 245.181981 79.818019) (end 246.5 83) (layer "Edge.Cuts") (width 0.1))
 (gr_line (start 191.5 78.5) (end 242 78.5) (layer "Edge.Cuts") (width 0.1))
 (gr_line (start 246.5 83) (end 246.5 122) (layer "Edge.Cuts") (width 0.1))
 (gr_arc (start 188 130) (mid 184.81802 128.681981) (end 183.5 125.5) (layer "Edge.Cuts") (width 0.1))
 (gr_line (start 238.5 130) (end 246.5 122) (layer "Edge.Cuts") (width 0.1))
 (segment (start 225.485858 122.485858) (end 229.111846 122.485858) (width 0.75) (layer "F.Cu") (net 9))
 (segment (start 195.25 110.63) (end 199.88 110.63) (width 0.75) (layer "F.Cu") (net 9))
 (segment (start 221.5 118.5) (end 238 102) (width 0.75) (layer "F.Cu") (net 9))
 (segment (start 207.75 118.5) (end 221.5 118.5) (width 0.75) (layer "F.Cu") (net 9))
 (segment (start 238 102) (end 241 102) (width 0.75) (layer "F.Cu") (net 9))
 (segment (start 199.88 110.63) (end 207.75 118.5) (width 0.75) (layer "F.Cu") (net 9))
 (segment (start 221.5 118.5) (end 225.485858 122.485858) (width 0.75) (layer "F.Cu") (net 9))
 (segment (start 229.861736 81) (end 227 81) (width 0.75) (layer "B.Cu") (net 9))
 (segment (start 227 81) (end 207.125 100.875) (width 0.75) (layer "B.Cu") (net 9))
 (segment (start 189.375 100.875) (end 185.979999 104.270001) (width 0.75) (layer "B.Cu") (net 9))
 (segment (start 230.180868 81.319132) (end 229.861736 81) (width 0.75) (layer "B.Cu") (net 9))
 (segment (start 195.25 110.63) (end 186.124999 110.63) (width 0.75) (layer "B.Cu") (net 9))
 (segment (start 186.124999 110.63) (end 185.979999 110.485) (width 0.75) (layer "B.Cu") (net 9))
 (segment (start 185.979999 104.270001) (end 185.979999 110.485) (width 0.75) (layer "B.Cu") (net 9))
 (segment (start 207.125 100.875) (end 189.375 100.875) (width 0.75) (layer "B.Cu") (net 9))
 (segment (start 195.110913 119.042894) (end 199.707107 123.639088) (width 0.75) (layer "F.Cu") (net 2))
 (segment (start 190.5 102.125001) (end 185.979999 97.605) (width 0.75) (layer "F.Cu") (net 2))
 (segment (start 190.5 103) (end 192 103) (width 0.75) (layer "F.Cu") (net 2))
 (segment (start 200 88.25) (end 230.240883 88.25) (width 0.75) (layer "F.Cu") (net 2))
 (segment (start 197.75 86) (end 200 88.25) (width 0.75) (layer "F.Cu") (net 2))
 (segment (start 185.979999 94.020001) (end 185.979999 97.605) (width 0.75) (layer "F.Cu") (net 2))
 (segment (start 193 116.931981) (end 193 104) (width 0.75) (layer "F.Cu") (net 2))
 (segment (start 230.240883 88.25) (end 230.811882 87.679001) (width 0.75) (layer "F.Cu") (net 2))
 (segment (start 192 103) (end 193 104) (width 0.75) (layer "F.Cu") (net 2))
 (segment (start 199.707107 123.639088) (end 199.707107 124.207107) (width 0.75) (layer "F.Cu") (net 2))
 (segment (start 191.5 88.5) (end 194 86) (width 0.75) (layer "F.Cu") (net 2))
 (segment (start 199.707107 124.207107) (end 202 126.5) (width 0.75) (layer "F.Cu") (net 2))
 (segment (start 194 86) (end 197.75 86) (width 0.75) (layer "F.Cu") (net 2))
 (segment (start 190.5 103) (end 190.5 102.125001) (width 0.75) (layer "F.Cu") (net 2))
 (segment (start 195.110913 119.042894) (end 193 116.931981) (width 0.75) (layer "F.Cu") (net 2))
 (segment (start 191.5 88.5) (end 185.979999 94.020001) (width 0.75) (layer "F.Cu") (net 2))
 (segment (start 234.5 119.5) (end 235.106244 118.893756) (width 0.75) (layer "B.Cu") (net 2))
 (segment (start 235.106244 118.893756) (end 235.856244 118.893756) (width 0.75) (layer "B.Cu") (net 2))
 (segment (start 235.856244 118.893756) (end 237.5 117.25) (width 0.75) (layer "B.Cu") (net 2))
 (segment (start 230.811882 105.811882) (end 230.811882 87.679001) (width 0.75) (layer "B.Cu") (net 2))
 (segment (start 234.5 119.5) (end 233.893756 118.893756) (width 0.75) (layer "B.Cu") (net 2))
 (segment (start 234.5 127.874012) (end 234.5 120) (width 0.75) (layer "B.Cu") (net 2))
 (segment (start 234.5 120) (end 234.5 119.5) (width 0.75) (layer "B.Cu") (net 2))
 (segment (start 237.5 112.5) (end 230.811882 105.811882) (width 0.75) (layer "B.Cu") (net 2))
 (segment (start 233.893756 118.893756) (end 235.106244 118.893756) (width 0.75) (layer "B.Cu") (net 2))
 (segment (start 232.703949 118.893756) (end 233.893756 118.893756) (width 0.75) (layer "B.Cu") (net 2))
 (segment (start 237.5 117.25) (end 237.5 112.5) (width 0.75) (layer "B.Cu") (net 2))
 (segment (start 228.384817 83.115183) (end 229.840166 83.115183) (width 0.75) (layer "F.Cu") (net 3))
 (segment (start 229.840166 83.115183) (end 232.607933 85.88295) (width 0.75) (layer "F.Cu") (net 3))
 (segment (start 206 105.5) (end 203.5 105.5) (width 0.75) (layer "B.Cu") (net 3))
 (segment (start 190.5 105.5) (end 203.5 105.5) (width 0.75) (layer "B.Cu") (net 3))
 (segment (start 228.384817 83.115183) (end 206 105.5) (width 0.75) (layer "B.Cu") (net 3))
 (segment (start 225.75 121.25) (end 230.25 116.75) (width 0.75) (layer "B.Cu") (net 7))
 (segment (start 207 126.5) (end 212.25 121.25) (width 0.75) (layer "B.Cu") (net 7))
 (segment (start 234.152295 116.75) (end 234.5 117.097705) (width 0.75) (layer "B.Cu") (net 7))
 (segment (start 230.25 116.75) (end 234.152295 116.75) (width 0.75) (layer "B.Cu") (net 7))
 (segment (start 212.25 121.25) (end 225.75 121.25) (width 0.75) (layer "B.Cu") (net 7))
 (segment (start 190.83 93.17) (end 194.04 89.96) (width 0.75) (layer "F.Cu") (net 10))
 (segment (start 190.83 94.5) (end 190.83 93.17) (width 0.75) (layer "F.Cu") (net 10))
 (segment (start 194.04 89.96) (end 194.04 88.5) (width 0.75) (layer "F.Cu") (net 10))
 (segment (start 239.888154 122.485858) (end 239.888154 114.888154) (width 0.75) (layer "F.Cu") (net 1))
 (segment (start 239.888154 114.888154) (end 239.5 114.5) (width 0.75) (layer "F.Cu") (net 1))
 (segment (start 241 107) (end 241 113) (width 0.75) (layer "B.Cu") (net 1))
 (segment (start 241 113) (end 239.5 114.5) (width 0.75) (layer "B.Cu") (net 1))
 (segment (start 233.819132 93.180868) (end 233 92.361736) (width 0.75) (layer "B.Cu") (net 4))
 (segment (start 233 88.071069) (end 231.709907 86.780976) (width 0.75) (layer "B.Cu") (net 4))
 (segment (start 233 92.361736) (end 233 88.071069) (width 0.75) (layer "B.Cu") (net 4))
 (segment (start 236.75 126) (end 229.75 126) (width 0.75) (layer "F.Cu") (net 6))
 (segment (start 229.75 126) (end 228.25 127.5) (width 0.75) (layer "F.Cu") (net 6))
 (segment (start 198.292894 115.860913) (end 202.889088 120.457107) (width 0.75) (layer "F.Cu") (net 6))
 (segment (start 198.292893 115.860913) (end 197.940913 115.860913) (width 0.75) (layer "F.Cu") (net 6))
 (segment (start 212.5 127.5) (end 205.457107 120.457107) (width 0.75) (layer "F.Cu") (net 6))
 (segment (start 197.940913 115.860913) (end 195.25 113.17) (width 0.75) (layer "F.Cu") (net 6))
 (segment (start 205.457107 120.457107) (end 202.889088 120.457107) (width 0.75) (layer "F.Cu") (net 6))
 (segment (start 228.25 127.5) (end 212.5 127.5) (width 0.75) (layer "F.Cu") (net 6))
 (segment (start 198.292893 115.860913) (end 198.292894 115.860913) (width 0.75) (layer "F.Cu") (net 6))
 (segment (start 244.5 95.973583) (end 239.911234 91.384817) (width 0.75) (layer "F.Cu") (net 5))
 (segment (start 206.25 90.5) (end 229.5 90.5) (width 0.75) (layer "F.Cu") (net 5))
 (segment (start 238.310192 124.5) (end 241.5 124.5) (width 0.75) (layer "F.Cu") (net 5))
 (segment (start 201 95.75) (end 206.25 90.5) (width 0.75) (layer "F.Cu") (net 5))
 (segment (start 193.37 94.5) (end 194.75 94.5) (width 0.75) (layer "F.Cu") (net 5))
 (segment (start 244.5 113.5) (end 244.5 95.973583) (width 0.75) (layer "F.Cu") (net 5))
 (segment (start 239.911234 91.384817) (end 235.615183 91.384817) (width 0.75) (layer "F.Cu") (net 5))
 (segment (start 194.75 94.5) (end 196 95.75) (width 0.75) (layer "F.Cu") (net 5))
 (segment (start 196 95.75) (end 201 95.75) (width 0.75) (layer "F.Cu") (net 5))
 (segment (start 238.092102 124.28191) (end 238.310192 124.5) (width 0.75) (layer "F.Cu") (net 5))
 (segment (start 242.5 123.5) (end 242.5 115.5) (width 0.75) (layer "F.Cu") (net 5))
 (segment (start 241.5 124.5) (end 242.5 123.5) (width 0.75) (layer "F.Cu") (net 5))
 (segment (start 229.5 90.5) (end 230.384817 91.384817) (width 0.75) (layer "F.Cu") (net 5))
 (segment (start 242.5 115.5) (end 244.5 113.5) (width 0.75) (layer "F.Cu") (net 5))
 (segment (start 230.384817 91.384817) (end 235.615183 91.384817) (width 0.75) (layer "F.Cu") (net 5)))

